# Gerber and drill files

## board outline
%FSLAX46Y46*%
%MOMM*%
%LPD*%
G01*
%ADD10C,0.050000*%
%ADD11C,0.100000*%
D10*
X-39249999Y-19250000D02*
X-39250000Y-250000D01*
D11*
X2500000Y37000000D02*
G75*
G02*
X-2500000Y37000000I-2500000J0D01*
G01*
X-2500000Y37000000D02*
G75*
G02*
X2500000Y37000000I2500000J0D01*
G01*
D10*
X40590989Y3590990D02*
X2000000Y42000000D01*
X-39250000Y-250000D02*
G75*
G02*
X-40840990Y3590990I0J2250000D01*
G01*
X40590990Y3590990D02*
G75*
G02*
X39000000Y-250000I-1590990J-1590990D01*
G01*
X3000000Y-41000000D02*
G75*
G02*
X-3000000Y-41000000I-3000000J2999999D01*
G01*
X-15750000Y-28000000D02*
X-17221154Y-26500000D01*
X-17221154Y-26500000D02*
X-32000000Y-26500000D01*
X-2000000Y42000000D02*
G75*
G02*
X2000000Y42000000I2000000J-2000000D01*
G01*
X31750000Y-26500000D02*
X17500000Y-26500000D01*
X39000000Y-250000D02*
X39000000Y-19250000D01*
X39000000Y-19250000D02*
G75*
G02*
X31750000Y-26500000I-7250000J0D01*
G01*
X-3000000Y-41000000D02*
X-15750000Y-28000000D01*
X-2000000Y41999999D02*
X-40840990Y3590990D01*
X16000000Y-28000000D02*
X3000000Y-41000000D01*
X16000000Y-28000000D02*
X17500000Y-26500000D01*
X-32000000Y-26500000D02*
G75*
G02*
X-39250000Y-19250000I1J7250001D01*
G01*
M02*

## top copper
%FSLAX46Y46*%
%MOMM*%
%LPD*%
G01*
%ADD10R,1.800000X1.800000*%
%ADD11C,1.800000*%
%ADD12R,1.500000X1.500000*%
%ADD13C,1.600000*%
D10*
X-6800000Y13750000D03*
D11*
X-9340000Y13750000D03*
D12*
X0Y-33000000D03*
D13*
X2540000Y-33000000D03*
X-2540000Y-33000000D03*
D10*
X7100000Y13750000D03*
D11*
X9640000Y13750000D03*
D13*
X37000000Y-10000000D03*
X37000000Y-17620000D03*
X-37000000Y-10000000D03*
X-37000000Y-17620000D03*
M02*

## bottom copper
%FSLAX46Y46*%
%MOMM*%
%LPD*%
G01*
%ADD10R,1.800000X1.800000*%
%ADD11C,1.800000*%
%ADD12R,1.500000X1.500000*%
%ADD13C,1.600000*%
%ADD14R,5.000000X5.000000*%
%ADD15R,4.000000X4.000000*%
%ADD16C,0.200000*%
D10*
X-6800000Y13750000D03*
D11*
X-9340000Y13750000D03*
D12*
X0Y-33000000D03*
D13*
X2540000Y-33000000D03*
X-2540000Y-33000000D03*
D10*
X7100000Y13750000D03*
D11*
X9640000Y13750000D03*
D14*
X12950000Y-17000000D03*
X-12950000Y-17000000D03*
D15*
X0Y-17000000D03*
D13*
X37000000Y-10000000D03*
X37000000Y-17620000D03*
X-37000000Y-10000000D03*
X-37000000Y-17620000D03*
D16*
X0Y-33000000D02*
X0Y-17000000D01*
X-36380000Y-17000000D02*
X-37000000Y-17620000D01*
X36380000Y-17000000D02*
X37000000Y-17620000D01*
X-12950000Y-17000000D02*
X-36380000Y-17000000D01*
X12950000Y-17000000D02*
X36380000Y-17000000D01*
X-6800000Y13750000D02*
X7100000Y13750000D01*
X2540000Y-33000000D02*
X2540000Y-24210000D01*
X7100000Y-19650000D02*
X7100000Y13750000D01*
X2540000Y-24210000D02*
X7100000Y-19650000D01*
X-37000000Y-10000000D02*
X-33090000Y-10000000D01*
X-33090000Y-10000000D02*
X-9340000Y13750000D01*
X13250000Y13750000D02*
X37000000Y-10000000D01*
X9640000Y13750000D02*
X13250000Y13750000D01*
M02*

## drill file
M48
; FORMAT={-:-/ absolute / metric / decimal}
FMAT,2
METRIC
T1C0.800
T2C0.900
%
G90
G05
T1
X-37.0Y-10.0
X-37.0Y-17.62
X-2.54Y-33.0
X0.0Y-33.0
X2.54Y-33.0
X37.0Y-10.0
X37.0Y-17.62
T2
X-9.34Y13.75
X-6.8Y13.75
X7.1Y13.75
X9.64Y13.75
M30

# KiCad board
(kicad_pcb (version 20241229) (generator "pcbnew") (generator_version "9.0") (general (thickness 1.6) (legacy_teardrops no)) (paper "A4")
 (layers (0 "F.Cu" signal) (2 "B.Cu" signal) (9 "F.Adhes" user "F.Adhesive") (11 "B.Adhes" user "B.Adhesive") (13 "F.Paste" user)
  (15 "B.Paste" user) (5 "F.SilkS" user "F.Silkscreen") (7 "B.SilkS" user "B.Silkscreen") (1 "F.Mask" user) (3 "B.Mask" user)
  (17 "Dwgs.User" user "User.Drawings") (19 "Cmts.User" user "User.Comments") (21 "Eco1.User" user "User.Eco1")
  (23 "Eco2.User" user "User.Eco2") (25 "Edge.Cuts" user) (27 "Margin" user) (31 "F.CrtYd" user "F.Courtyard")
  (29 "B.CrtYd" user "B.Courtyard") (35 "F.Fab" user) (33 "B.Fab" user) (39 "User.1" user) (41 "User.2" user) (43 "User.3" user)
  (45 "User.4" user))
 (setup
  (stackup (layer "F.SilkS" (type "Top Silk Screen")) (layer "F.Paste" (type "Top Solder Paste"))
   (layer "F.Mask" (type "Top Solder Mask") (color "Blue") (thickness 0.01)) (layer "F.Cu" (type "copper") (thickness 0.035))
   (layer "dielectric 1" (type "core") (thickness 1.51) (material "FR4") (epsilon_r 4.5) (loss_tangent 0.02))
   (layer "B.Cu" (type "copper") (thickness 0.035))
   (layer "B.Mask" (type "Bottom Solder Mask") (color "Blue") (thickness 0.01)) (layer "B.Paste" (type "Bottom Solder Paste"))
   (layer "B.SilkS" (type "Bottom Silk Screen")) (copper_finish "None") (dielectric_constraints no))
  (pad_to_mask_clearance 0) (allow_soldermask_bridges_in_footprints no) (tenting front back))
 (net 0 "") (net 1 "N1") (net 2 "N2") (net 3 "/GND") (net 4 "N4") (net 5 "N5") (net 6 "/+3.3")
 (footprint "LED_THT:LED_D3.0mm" (layer "F.Cu") (at -6.8 -13.75 180)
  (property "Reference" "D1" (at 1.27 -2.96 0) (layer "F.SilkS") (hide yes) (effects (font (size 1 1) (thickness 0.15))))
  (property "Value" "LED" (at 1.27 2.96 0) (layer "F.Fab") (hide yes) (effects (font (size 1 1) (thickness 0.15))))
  (pad "1" thru_hole rect (at 0 0 180) (size 1.8 1.8) (drill 0.9) (layers "*.Cu" "*.Mask") (remove_unused_layers no) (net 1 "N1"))
  (pad "2" thru_hole circle (at 2.54 0 180) (size 1.8 1.8) (drill 0.9) (layers "*.Cu" "*.Mask") (remove_unused_layers no) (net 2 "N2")))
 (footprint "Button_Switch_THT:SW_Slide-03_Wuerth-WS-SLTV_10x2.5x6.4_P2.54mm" (layer "F.Cu") (at 0 33 180)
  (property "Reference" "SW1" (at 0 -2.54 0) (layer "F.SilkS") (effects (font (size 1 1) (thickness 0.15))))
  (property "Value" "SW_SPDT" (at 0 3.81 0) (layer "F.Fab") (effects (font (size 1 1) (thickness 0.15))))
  (pad "1" thru_hole rect (at 0 0 180) (size 1.5 1.5) (drill 0.8) (layers "*.Cu" "*.Mask") (remove_unused_layers no) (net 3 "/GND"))
  (pad "2" thru_hole circle (at -2.54 0 180) (size 1.6 1.6) (drill 0.8) (layers "*.Cu" "*.Mask") (remove_unused_layers no) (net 1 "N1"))
  (pad "3" thru_hole circle (at 2.54 0 180) (size 1.6 1.6) (drill 0.8) (layers "*.Cu" "*.Mask") (remove_unused_layers no) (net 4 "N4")))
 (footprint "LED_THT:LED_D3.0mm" (layer "F.Cu") (at 7.1 -13.75)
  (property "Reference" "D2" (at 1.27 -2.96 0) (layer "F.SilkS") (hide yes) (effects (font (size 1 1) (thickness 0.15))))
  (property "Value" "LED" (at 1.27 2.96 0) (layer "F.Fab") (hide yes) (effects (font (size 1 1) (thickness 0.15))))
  (pad "1" thru_hole rect (at 0 0) (size 1.8 1.8) (drill 0.9) (layers "*.Cu" "*.Mask") (remove_unused_layers no) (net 1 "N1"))
  (pad "2" thru_hole circle (at 2.54 0) (size 1.8 1.8) (drill 0.9) (layers "*.Cu" "*.Mask") (remove_unused_layers no) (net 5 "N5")))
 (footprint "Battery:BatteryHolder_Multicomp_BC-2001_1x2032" (layer "B.Cu") (at 0 17 180)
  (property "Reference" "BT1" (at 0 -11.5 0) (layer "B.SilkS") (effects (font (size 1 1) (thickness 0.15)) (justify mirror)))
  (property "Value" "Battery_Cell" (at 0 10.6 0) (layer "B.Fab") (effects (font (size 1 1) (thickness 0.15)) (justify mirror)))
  (pad "1" smd rect (at -12.95 0 180) (size 5 5) (layers "B.Cu" "B.Mask" "B.Paste") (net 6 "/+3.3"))
  (pad "1" smd rect (at 12.95 0 180) (size 5 5) (layers "B.Cu" "B.Mask" "B.Paste") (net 6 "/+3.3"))
  (pad "2" smd rect (at 0 0 180) (size 4 4) (layers "B.Cu" "B.Mask" "B.Paste") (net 3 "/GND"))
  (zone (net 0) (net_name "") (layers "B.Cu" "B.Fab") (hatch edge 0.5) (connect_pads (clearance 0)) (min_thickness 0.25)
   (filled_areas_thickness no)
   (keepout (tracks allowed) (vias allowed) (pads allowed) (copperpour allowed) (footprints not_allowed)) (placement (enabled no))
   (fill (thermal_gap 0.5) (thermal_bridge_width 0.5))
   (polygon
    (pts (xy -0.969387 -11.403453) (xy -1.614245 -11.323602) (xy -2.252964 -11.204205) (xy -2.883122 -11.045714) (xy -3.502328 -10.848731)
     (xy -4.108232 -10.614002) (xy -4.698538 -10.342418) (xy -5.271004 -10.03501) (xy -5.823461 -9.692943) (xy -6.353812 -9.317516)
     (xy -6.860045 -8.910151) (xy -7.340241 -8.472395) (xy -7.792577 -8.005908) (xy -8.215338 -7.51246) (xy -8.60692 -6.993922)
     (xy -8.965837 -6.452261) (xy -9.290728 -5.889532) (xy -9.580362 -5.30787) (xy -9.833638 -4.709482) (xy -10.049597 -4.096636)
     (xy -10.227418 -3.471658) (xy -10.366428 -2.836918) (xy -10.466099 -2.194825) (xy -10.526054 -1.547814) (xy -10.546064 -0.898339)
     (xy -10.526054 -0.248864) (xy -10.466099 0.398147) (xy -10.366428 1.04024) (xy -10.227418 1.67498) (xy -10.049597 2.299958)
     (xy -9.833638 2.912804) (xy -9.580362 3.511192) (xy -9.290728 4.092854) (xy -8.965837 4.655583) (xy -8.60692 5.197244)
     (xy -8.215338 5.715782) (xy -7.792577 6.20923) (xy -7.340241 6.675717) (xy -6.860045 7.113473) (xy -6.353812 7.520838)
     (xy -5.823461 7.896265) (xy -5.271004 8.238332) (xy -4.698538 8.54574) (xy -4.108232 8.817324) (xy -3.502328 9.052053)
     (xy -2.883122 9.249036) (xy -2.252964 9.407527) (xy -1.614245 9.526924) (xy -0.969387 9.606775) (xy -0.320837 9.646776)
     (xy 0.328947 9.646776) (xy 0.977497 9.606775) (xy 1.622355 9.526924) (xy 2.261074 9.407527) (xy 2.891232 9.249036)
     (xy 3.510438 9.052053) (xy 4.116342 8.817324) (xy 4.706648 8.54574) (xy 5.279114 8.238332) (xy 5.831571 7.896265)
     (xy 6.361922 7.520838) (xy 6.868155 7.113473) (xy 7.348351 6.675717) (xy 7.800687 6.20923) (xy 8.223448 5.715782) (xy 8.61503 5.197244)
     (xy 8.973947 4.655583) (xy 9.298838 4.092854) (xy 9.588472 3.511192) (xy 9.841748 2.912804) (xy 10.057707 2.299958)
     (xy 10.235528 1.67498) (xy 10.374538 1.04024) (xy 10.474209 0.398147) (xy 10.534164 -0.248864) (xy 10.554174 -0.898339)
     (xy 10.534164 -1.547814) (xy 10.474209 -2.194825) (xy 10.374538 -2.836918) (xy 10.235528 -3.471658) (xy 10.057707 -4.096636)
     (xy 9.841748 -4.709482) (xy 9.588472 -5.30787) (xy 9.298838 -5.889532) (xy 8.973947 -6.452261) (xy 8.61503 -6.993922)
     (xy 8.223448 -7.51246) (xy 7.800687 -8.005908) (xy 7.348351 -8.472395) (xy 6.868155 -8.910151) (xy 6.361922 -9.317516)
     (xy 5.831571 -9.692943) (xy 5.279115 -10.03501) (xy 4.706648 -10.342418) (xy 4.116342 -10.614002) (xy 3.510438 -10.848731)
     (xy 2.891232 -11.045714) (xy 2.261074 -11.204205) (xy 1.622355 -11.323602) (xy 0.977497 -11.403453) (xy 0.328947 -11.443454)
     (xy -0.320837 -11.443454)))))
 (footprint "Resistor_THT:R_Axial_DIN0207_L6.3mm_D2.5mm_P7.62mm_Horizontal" (layer "B.Cu") (at 37 10 -90)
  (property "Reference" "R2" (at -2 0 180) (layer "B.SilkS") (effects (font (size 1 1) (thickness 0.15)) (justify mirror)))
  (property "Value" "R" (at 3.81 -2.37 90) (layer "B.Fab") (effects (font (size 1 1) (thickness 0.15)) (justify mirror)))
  (pad "1" thru_hole circle (at 0 0 270) (size 1.6 1.6) (drill 0.8) (layers "*.Cu" "*.Mask") (remove_unused_layers no) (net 5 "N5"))
  (pad "2" thru_hole circle (at 7.62 0 270) (size 1.6 1.6) (drill 0.8) (layers "*.Cu" "*.Mask") (remove_unused_layers no) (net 6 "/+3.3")))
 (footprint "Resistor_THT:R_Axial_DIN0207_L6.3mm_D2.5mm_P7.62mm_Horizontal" (layer "B.Cu") (at -37 10 -90)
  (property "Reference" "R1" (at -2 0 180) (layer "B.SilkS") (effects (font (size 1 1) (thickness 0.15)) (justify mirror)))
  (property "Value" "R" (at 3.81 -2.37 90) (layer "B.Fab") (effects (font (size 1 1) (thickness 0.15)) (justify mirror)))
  (pad "1" thru_hole circle (at 0 0 270) (size 1.6 1.6) (drill 0.8) (layers "*.Cu" "*.Mask") (remove_unused_layers no) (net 2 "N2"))
  (pad "2" thru_hole circle (at 7.62 0 270) (size 1.6 1.6) (drill 0.8) (layers "*.Cu" "*.Mask") (remove_unused_layers no) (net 6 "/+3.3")))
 (gr_line (start -39.249999 19.25) (end -39.25 0.25) (stroke (width 0.05) (type default)) (layer "Edge.Cuts"))
 (gr_circle (center 0 -37) (end 2.5 -37) (stroke (width 0.1) (type solid)) (fill no) (layer "Edge.Cuts"))
 (gr_line (start 40.590989 -3.59099) (end 2 -42) (stroke (width 0.05) (type default)) (layer "Edge.Cuts"))
 (gr_arc (start -39.25 0.25) (mid -41.328729 -1.138962) (end -40.84099 -3.59099) (stroke (width 0.05) (type default)) (layer "Edge.Cuts"))
 (gr_arc (start 40.59099 -3.59099) (mid 41.078729 -1.138962) (end 39 0.25) (stroke (width 0.05) (type default)) (layer "Edge.Cuts"))
 (gr_arc (start 3 41) (mid 0 42.242641) (end -3 41) (stroke (width 0.05) (type default)) (layer "Edge.Cuts"))
 (gr_line (start -15.75 28) (end -17.221154 26.5) (stroke (width 0.05) (type default)) (layer "Edge.Cuts"))
 (gr_line (start -17.221154 26.5) (end -32 26.5) (stroke (width 0.05) (type default)) (layer "Edge.Cuts"))
 (gr_arc (start -2 -42) (mid 0 -42.828427) (end 2 -42) (stroke (width 0.05) (type default)) (layer "Edge.Cuts"))
 (gr_line (start 31.75 26.5) (end 17.5 26.5) (stroke (width 0.05) (type default)) (layer "Edge.Cuts"))
 (gr_line (start 39 0.25) (end 39 19.25) (stroke (width 0.05) (type default)) (layer "Edge.Cuts"))
 (gr_arc (start 39 19.25) (mid 36.876524 24.376524) (end 31.75 26.5) (stroke (width 0.05) (type default)) (layer "Edge.Cuts"))
 (gr_line (start -3 41) (end -15.75 28) (stroke (width 0.05) (type default)) (layer "Edge.Cuts"))
 (gr_line (start -2 -41.999999) (end -40.84099 -3.59099) (stroke (width 0.05) (type default)) (layer "Edge.Cuts"))
 (gr_line (start 16 28) (end 3 41) (stroke (width 0.05) (type default)) (layer "Edge.Cuts"))
 (gr_line (start 16 28) (end 17.5 26.5) (stroke (width 0.05) (type default)) (layer "Edge.Cuts"))
 (gr_arc (start -32 26.5) (mid -37.126524 24.376524) (end -39.25 19.25) (stroke (width 0.05) (type default)) (layer "Edge.Cuts"))
 (segment (start 0 33) (end 0 17) (width 0.2) (layer "B.Cu") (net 3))
 (segment (start -36.38 17) (end -37 17.62) (width 0.2) (layer "B.Cu") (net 6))
 (segment (start 36.38 17) (end 37 17.62) (width 0.2) (layer "B.Cu") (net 6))
 (segment (start -12.95 17) (end -36.38 17) (width 0.2) (layer "B.Cu") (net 6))
 (segment (start 12.95 17) (end 36.38 17) (width 0.2) (layer "B.Cu") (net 6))
 (segment (start -6.8 -13.75) (end 7.1 -13.75) (width 0.2) (layer "B.Cu") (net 1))
 (segment (start 2.54 33) (end 2.54 24.21) (width 0.2) (layer "B.Cu") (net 1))
 (segment (start 7.1 19.65) (end 7.1 -13.75) (width 0.2) (layer "B.Cu") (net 1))
 (segment (start 2.54 24.21) (end 7.1 19.65) (width 0.2) (layer "B.Cu") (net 1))
 (segment (start -37 10) (end -33.09 10) (width 0.2) (layer "B.Cu") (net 2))
 (segment (start -33.09 10) (end -9.34 -13.75) (width 0.2) (layer "B.Cu") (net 2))
 (segment (start 13.25 -13.75) (end 37 10) (width 0.2) (layer "B.Cu") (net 5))
 (segment (start 9.64 -13.75) (end 13.25 -13.75) (width 0.2) (layer "B.Cu") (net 5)))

